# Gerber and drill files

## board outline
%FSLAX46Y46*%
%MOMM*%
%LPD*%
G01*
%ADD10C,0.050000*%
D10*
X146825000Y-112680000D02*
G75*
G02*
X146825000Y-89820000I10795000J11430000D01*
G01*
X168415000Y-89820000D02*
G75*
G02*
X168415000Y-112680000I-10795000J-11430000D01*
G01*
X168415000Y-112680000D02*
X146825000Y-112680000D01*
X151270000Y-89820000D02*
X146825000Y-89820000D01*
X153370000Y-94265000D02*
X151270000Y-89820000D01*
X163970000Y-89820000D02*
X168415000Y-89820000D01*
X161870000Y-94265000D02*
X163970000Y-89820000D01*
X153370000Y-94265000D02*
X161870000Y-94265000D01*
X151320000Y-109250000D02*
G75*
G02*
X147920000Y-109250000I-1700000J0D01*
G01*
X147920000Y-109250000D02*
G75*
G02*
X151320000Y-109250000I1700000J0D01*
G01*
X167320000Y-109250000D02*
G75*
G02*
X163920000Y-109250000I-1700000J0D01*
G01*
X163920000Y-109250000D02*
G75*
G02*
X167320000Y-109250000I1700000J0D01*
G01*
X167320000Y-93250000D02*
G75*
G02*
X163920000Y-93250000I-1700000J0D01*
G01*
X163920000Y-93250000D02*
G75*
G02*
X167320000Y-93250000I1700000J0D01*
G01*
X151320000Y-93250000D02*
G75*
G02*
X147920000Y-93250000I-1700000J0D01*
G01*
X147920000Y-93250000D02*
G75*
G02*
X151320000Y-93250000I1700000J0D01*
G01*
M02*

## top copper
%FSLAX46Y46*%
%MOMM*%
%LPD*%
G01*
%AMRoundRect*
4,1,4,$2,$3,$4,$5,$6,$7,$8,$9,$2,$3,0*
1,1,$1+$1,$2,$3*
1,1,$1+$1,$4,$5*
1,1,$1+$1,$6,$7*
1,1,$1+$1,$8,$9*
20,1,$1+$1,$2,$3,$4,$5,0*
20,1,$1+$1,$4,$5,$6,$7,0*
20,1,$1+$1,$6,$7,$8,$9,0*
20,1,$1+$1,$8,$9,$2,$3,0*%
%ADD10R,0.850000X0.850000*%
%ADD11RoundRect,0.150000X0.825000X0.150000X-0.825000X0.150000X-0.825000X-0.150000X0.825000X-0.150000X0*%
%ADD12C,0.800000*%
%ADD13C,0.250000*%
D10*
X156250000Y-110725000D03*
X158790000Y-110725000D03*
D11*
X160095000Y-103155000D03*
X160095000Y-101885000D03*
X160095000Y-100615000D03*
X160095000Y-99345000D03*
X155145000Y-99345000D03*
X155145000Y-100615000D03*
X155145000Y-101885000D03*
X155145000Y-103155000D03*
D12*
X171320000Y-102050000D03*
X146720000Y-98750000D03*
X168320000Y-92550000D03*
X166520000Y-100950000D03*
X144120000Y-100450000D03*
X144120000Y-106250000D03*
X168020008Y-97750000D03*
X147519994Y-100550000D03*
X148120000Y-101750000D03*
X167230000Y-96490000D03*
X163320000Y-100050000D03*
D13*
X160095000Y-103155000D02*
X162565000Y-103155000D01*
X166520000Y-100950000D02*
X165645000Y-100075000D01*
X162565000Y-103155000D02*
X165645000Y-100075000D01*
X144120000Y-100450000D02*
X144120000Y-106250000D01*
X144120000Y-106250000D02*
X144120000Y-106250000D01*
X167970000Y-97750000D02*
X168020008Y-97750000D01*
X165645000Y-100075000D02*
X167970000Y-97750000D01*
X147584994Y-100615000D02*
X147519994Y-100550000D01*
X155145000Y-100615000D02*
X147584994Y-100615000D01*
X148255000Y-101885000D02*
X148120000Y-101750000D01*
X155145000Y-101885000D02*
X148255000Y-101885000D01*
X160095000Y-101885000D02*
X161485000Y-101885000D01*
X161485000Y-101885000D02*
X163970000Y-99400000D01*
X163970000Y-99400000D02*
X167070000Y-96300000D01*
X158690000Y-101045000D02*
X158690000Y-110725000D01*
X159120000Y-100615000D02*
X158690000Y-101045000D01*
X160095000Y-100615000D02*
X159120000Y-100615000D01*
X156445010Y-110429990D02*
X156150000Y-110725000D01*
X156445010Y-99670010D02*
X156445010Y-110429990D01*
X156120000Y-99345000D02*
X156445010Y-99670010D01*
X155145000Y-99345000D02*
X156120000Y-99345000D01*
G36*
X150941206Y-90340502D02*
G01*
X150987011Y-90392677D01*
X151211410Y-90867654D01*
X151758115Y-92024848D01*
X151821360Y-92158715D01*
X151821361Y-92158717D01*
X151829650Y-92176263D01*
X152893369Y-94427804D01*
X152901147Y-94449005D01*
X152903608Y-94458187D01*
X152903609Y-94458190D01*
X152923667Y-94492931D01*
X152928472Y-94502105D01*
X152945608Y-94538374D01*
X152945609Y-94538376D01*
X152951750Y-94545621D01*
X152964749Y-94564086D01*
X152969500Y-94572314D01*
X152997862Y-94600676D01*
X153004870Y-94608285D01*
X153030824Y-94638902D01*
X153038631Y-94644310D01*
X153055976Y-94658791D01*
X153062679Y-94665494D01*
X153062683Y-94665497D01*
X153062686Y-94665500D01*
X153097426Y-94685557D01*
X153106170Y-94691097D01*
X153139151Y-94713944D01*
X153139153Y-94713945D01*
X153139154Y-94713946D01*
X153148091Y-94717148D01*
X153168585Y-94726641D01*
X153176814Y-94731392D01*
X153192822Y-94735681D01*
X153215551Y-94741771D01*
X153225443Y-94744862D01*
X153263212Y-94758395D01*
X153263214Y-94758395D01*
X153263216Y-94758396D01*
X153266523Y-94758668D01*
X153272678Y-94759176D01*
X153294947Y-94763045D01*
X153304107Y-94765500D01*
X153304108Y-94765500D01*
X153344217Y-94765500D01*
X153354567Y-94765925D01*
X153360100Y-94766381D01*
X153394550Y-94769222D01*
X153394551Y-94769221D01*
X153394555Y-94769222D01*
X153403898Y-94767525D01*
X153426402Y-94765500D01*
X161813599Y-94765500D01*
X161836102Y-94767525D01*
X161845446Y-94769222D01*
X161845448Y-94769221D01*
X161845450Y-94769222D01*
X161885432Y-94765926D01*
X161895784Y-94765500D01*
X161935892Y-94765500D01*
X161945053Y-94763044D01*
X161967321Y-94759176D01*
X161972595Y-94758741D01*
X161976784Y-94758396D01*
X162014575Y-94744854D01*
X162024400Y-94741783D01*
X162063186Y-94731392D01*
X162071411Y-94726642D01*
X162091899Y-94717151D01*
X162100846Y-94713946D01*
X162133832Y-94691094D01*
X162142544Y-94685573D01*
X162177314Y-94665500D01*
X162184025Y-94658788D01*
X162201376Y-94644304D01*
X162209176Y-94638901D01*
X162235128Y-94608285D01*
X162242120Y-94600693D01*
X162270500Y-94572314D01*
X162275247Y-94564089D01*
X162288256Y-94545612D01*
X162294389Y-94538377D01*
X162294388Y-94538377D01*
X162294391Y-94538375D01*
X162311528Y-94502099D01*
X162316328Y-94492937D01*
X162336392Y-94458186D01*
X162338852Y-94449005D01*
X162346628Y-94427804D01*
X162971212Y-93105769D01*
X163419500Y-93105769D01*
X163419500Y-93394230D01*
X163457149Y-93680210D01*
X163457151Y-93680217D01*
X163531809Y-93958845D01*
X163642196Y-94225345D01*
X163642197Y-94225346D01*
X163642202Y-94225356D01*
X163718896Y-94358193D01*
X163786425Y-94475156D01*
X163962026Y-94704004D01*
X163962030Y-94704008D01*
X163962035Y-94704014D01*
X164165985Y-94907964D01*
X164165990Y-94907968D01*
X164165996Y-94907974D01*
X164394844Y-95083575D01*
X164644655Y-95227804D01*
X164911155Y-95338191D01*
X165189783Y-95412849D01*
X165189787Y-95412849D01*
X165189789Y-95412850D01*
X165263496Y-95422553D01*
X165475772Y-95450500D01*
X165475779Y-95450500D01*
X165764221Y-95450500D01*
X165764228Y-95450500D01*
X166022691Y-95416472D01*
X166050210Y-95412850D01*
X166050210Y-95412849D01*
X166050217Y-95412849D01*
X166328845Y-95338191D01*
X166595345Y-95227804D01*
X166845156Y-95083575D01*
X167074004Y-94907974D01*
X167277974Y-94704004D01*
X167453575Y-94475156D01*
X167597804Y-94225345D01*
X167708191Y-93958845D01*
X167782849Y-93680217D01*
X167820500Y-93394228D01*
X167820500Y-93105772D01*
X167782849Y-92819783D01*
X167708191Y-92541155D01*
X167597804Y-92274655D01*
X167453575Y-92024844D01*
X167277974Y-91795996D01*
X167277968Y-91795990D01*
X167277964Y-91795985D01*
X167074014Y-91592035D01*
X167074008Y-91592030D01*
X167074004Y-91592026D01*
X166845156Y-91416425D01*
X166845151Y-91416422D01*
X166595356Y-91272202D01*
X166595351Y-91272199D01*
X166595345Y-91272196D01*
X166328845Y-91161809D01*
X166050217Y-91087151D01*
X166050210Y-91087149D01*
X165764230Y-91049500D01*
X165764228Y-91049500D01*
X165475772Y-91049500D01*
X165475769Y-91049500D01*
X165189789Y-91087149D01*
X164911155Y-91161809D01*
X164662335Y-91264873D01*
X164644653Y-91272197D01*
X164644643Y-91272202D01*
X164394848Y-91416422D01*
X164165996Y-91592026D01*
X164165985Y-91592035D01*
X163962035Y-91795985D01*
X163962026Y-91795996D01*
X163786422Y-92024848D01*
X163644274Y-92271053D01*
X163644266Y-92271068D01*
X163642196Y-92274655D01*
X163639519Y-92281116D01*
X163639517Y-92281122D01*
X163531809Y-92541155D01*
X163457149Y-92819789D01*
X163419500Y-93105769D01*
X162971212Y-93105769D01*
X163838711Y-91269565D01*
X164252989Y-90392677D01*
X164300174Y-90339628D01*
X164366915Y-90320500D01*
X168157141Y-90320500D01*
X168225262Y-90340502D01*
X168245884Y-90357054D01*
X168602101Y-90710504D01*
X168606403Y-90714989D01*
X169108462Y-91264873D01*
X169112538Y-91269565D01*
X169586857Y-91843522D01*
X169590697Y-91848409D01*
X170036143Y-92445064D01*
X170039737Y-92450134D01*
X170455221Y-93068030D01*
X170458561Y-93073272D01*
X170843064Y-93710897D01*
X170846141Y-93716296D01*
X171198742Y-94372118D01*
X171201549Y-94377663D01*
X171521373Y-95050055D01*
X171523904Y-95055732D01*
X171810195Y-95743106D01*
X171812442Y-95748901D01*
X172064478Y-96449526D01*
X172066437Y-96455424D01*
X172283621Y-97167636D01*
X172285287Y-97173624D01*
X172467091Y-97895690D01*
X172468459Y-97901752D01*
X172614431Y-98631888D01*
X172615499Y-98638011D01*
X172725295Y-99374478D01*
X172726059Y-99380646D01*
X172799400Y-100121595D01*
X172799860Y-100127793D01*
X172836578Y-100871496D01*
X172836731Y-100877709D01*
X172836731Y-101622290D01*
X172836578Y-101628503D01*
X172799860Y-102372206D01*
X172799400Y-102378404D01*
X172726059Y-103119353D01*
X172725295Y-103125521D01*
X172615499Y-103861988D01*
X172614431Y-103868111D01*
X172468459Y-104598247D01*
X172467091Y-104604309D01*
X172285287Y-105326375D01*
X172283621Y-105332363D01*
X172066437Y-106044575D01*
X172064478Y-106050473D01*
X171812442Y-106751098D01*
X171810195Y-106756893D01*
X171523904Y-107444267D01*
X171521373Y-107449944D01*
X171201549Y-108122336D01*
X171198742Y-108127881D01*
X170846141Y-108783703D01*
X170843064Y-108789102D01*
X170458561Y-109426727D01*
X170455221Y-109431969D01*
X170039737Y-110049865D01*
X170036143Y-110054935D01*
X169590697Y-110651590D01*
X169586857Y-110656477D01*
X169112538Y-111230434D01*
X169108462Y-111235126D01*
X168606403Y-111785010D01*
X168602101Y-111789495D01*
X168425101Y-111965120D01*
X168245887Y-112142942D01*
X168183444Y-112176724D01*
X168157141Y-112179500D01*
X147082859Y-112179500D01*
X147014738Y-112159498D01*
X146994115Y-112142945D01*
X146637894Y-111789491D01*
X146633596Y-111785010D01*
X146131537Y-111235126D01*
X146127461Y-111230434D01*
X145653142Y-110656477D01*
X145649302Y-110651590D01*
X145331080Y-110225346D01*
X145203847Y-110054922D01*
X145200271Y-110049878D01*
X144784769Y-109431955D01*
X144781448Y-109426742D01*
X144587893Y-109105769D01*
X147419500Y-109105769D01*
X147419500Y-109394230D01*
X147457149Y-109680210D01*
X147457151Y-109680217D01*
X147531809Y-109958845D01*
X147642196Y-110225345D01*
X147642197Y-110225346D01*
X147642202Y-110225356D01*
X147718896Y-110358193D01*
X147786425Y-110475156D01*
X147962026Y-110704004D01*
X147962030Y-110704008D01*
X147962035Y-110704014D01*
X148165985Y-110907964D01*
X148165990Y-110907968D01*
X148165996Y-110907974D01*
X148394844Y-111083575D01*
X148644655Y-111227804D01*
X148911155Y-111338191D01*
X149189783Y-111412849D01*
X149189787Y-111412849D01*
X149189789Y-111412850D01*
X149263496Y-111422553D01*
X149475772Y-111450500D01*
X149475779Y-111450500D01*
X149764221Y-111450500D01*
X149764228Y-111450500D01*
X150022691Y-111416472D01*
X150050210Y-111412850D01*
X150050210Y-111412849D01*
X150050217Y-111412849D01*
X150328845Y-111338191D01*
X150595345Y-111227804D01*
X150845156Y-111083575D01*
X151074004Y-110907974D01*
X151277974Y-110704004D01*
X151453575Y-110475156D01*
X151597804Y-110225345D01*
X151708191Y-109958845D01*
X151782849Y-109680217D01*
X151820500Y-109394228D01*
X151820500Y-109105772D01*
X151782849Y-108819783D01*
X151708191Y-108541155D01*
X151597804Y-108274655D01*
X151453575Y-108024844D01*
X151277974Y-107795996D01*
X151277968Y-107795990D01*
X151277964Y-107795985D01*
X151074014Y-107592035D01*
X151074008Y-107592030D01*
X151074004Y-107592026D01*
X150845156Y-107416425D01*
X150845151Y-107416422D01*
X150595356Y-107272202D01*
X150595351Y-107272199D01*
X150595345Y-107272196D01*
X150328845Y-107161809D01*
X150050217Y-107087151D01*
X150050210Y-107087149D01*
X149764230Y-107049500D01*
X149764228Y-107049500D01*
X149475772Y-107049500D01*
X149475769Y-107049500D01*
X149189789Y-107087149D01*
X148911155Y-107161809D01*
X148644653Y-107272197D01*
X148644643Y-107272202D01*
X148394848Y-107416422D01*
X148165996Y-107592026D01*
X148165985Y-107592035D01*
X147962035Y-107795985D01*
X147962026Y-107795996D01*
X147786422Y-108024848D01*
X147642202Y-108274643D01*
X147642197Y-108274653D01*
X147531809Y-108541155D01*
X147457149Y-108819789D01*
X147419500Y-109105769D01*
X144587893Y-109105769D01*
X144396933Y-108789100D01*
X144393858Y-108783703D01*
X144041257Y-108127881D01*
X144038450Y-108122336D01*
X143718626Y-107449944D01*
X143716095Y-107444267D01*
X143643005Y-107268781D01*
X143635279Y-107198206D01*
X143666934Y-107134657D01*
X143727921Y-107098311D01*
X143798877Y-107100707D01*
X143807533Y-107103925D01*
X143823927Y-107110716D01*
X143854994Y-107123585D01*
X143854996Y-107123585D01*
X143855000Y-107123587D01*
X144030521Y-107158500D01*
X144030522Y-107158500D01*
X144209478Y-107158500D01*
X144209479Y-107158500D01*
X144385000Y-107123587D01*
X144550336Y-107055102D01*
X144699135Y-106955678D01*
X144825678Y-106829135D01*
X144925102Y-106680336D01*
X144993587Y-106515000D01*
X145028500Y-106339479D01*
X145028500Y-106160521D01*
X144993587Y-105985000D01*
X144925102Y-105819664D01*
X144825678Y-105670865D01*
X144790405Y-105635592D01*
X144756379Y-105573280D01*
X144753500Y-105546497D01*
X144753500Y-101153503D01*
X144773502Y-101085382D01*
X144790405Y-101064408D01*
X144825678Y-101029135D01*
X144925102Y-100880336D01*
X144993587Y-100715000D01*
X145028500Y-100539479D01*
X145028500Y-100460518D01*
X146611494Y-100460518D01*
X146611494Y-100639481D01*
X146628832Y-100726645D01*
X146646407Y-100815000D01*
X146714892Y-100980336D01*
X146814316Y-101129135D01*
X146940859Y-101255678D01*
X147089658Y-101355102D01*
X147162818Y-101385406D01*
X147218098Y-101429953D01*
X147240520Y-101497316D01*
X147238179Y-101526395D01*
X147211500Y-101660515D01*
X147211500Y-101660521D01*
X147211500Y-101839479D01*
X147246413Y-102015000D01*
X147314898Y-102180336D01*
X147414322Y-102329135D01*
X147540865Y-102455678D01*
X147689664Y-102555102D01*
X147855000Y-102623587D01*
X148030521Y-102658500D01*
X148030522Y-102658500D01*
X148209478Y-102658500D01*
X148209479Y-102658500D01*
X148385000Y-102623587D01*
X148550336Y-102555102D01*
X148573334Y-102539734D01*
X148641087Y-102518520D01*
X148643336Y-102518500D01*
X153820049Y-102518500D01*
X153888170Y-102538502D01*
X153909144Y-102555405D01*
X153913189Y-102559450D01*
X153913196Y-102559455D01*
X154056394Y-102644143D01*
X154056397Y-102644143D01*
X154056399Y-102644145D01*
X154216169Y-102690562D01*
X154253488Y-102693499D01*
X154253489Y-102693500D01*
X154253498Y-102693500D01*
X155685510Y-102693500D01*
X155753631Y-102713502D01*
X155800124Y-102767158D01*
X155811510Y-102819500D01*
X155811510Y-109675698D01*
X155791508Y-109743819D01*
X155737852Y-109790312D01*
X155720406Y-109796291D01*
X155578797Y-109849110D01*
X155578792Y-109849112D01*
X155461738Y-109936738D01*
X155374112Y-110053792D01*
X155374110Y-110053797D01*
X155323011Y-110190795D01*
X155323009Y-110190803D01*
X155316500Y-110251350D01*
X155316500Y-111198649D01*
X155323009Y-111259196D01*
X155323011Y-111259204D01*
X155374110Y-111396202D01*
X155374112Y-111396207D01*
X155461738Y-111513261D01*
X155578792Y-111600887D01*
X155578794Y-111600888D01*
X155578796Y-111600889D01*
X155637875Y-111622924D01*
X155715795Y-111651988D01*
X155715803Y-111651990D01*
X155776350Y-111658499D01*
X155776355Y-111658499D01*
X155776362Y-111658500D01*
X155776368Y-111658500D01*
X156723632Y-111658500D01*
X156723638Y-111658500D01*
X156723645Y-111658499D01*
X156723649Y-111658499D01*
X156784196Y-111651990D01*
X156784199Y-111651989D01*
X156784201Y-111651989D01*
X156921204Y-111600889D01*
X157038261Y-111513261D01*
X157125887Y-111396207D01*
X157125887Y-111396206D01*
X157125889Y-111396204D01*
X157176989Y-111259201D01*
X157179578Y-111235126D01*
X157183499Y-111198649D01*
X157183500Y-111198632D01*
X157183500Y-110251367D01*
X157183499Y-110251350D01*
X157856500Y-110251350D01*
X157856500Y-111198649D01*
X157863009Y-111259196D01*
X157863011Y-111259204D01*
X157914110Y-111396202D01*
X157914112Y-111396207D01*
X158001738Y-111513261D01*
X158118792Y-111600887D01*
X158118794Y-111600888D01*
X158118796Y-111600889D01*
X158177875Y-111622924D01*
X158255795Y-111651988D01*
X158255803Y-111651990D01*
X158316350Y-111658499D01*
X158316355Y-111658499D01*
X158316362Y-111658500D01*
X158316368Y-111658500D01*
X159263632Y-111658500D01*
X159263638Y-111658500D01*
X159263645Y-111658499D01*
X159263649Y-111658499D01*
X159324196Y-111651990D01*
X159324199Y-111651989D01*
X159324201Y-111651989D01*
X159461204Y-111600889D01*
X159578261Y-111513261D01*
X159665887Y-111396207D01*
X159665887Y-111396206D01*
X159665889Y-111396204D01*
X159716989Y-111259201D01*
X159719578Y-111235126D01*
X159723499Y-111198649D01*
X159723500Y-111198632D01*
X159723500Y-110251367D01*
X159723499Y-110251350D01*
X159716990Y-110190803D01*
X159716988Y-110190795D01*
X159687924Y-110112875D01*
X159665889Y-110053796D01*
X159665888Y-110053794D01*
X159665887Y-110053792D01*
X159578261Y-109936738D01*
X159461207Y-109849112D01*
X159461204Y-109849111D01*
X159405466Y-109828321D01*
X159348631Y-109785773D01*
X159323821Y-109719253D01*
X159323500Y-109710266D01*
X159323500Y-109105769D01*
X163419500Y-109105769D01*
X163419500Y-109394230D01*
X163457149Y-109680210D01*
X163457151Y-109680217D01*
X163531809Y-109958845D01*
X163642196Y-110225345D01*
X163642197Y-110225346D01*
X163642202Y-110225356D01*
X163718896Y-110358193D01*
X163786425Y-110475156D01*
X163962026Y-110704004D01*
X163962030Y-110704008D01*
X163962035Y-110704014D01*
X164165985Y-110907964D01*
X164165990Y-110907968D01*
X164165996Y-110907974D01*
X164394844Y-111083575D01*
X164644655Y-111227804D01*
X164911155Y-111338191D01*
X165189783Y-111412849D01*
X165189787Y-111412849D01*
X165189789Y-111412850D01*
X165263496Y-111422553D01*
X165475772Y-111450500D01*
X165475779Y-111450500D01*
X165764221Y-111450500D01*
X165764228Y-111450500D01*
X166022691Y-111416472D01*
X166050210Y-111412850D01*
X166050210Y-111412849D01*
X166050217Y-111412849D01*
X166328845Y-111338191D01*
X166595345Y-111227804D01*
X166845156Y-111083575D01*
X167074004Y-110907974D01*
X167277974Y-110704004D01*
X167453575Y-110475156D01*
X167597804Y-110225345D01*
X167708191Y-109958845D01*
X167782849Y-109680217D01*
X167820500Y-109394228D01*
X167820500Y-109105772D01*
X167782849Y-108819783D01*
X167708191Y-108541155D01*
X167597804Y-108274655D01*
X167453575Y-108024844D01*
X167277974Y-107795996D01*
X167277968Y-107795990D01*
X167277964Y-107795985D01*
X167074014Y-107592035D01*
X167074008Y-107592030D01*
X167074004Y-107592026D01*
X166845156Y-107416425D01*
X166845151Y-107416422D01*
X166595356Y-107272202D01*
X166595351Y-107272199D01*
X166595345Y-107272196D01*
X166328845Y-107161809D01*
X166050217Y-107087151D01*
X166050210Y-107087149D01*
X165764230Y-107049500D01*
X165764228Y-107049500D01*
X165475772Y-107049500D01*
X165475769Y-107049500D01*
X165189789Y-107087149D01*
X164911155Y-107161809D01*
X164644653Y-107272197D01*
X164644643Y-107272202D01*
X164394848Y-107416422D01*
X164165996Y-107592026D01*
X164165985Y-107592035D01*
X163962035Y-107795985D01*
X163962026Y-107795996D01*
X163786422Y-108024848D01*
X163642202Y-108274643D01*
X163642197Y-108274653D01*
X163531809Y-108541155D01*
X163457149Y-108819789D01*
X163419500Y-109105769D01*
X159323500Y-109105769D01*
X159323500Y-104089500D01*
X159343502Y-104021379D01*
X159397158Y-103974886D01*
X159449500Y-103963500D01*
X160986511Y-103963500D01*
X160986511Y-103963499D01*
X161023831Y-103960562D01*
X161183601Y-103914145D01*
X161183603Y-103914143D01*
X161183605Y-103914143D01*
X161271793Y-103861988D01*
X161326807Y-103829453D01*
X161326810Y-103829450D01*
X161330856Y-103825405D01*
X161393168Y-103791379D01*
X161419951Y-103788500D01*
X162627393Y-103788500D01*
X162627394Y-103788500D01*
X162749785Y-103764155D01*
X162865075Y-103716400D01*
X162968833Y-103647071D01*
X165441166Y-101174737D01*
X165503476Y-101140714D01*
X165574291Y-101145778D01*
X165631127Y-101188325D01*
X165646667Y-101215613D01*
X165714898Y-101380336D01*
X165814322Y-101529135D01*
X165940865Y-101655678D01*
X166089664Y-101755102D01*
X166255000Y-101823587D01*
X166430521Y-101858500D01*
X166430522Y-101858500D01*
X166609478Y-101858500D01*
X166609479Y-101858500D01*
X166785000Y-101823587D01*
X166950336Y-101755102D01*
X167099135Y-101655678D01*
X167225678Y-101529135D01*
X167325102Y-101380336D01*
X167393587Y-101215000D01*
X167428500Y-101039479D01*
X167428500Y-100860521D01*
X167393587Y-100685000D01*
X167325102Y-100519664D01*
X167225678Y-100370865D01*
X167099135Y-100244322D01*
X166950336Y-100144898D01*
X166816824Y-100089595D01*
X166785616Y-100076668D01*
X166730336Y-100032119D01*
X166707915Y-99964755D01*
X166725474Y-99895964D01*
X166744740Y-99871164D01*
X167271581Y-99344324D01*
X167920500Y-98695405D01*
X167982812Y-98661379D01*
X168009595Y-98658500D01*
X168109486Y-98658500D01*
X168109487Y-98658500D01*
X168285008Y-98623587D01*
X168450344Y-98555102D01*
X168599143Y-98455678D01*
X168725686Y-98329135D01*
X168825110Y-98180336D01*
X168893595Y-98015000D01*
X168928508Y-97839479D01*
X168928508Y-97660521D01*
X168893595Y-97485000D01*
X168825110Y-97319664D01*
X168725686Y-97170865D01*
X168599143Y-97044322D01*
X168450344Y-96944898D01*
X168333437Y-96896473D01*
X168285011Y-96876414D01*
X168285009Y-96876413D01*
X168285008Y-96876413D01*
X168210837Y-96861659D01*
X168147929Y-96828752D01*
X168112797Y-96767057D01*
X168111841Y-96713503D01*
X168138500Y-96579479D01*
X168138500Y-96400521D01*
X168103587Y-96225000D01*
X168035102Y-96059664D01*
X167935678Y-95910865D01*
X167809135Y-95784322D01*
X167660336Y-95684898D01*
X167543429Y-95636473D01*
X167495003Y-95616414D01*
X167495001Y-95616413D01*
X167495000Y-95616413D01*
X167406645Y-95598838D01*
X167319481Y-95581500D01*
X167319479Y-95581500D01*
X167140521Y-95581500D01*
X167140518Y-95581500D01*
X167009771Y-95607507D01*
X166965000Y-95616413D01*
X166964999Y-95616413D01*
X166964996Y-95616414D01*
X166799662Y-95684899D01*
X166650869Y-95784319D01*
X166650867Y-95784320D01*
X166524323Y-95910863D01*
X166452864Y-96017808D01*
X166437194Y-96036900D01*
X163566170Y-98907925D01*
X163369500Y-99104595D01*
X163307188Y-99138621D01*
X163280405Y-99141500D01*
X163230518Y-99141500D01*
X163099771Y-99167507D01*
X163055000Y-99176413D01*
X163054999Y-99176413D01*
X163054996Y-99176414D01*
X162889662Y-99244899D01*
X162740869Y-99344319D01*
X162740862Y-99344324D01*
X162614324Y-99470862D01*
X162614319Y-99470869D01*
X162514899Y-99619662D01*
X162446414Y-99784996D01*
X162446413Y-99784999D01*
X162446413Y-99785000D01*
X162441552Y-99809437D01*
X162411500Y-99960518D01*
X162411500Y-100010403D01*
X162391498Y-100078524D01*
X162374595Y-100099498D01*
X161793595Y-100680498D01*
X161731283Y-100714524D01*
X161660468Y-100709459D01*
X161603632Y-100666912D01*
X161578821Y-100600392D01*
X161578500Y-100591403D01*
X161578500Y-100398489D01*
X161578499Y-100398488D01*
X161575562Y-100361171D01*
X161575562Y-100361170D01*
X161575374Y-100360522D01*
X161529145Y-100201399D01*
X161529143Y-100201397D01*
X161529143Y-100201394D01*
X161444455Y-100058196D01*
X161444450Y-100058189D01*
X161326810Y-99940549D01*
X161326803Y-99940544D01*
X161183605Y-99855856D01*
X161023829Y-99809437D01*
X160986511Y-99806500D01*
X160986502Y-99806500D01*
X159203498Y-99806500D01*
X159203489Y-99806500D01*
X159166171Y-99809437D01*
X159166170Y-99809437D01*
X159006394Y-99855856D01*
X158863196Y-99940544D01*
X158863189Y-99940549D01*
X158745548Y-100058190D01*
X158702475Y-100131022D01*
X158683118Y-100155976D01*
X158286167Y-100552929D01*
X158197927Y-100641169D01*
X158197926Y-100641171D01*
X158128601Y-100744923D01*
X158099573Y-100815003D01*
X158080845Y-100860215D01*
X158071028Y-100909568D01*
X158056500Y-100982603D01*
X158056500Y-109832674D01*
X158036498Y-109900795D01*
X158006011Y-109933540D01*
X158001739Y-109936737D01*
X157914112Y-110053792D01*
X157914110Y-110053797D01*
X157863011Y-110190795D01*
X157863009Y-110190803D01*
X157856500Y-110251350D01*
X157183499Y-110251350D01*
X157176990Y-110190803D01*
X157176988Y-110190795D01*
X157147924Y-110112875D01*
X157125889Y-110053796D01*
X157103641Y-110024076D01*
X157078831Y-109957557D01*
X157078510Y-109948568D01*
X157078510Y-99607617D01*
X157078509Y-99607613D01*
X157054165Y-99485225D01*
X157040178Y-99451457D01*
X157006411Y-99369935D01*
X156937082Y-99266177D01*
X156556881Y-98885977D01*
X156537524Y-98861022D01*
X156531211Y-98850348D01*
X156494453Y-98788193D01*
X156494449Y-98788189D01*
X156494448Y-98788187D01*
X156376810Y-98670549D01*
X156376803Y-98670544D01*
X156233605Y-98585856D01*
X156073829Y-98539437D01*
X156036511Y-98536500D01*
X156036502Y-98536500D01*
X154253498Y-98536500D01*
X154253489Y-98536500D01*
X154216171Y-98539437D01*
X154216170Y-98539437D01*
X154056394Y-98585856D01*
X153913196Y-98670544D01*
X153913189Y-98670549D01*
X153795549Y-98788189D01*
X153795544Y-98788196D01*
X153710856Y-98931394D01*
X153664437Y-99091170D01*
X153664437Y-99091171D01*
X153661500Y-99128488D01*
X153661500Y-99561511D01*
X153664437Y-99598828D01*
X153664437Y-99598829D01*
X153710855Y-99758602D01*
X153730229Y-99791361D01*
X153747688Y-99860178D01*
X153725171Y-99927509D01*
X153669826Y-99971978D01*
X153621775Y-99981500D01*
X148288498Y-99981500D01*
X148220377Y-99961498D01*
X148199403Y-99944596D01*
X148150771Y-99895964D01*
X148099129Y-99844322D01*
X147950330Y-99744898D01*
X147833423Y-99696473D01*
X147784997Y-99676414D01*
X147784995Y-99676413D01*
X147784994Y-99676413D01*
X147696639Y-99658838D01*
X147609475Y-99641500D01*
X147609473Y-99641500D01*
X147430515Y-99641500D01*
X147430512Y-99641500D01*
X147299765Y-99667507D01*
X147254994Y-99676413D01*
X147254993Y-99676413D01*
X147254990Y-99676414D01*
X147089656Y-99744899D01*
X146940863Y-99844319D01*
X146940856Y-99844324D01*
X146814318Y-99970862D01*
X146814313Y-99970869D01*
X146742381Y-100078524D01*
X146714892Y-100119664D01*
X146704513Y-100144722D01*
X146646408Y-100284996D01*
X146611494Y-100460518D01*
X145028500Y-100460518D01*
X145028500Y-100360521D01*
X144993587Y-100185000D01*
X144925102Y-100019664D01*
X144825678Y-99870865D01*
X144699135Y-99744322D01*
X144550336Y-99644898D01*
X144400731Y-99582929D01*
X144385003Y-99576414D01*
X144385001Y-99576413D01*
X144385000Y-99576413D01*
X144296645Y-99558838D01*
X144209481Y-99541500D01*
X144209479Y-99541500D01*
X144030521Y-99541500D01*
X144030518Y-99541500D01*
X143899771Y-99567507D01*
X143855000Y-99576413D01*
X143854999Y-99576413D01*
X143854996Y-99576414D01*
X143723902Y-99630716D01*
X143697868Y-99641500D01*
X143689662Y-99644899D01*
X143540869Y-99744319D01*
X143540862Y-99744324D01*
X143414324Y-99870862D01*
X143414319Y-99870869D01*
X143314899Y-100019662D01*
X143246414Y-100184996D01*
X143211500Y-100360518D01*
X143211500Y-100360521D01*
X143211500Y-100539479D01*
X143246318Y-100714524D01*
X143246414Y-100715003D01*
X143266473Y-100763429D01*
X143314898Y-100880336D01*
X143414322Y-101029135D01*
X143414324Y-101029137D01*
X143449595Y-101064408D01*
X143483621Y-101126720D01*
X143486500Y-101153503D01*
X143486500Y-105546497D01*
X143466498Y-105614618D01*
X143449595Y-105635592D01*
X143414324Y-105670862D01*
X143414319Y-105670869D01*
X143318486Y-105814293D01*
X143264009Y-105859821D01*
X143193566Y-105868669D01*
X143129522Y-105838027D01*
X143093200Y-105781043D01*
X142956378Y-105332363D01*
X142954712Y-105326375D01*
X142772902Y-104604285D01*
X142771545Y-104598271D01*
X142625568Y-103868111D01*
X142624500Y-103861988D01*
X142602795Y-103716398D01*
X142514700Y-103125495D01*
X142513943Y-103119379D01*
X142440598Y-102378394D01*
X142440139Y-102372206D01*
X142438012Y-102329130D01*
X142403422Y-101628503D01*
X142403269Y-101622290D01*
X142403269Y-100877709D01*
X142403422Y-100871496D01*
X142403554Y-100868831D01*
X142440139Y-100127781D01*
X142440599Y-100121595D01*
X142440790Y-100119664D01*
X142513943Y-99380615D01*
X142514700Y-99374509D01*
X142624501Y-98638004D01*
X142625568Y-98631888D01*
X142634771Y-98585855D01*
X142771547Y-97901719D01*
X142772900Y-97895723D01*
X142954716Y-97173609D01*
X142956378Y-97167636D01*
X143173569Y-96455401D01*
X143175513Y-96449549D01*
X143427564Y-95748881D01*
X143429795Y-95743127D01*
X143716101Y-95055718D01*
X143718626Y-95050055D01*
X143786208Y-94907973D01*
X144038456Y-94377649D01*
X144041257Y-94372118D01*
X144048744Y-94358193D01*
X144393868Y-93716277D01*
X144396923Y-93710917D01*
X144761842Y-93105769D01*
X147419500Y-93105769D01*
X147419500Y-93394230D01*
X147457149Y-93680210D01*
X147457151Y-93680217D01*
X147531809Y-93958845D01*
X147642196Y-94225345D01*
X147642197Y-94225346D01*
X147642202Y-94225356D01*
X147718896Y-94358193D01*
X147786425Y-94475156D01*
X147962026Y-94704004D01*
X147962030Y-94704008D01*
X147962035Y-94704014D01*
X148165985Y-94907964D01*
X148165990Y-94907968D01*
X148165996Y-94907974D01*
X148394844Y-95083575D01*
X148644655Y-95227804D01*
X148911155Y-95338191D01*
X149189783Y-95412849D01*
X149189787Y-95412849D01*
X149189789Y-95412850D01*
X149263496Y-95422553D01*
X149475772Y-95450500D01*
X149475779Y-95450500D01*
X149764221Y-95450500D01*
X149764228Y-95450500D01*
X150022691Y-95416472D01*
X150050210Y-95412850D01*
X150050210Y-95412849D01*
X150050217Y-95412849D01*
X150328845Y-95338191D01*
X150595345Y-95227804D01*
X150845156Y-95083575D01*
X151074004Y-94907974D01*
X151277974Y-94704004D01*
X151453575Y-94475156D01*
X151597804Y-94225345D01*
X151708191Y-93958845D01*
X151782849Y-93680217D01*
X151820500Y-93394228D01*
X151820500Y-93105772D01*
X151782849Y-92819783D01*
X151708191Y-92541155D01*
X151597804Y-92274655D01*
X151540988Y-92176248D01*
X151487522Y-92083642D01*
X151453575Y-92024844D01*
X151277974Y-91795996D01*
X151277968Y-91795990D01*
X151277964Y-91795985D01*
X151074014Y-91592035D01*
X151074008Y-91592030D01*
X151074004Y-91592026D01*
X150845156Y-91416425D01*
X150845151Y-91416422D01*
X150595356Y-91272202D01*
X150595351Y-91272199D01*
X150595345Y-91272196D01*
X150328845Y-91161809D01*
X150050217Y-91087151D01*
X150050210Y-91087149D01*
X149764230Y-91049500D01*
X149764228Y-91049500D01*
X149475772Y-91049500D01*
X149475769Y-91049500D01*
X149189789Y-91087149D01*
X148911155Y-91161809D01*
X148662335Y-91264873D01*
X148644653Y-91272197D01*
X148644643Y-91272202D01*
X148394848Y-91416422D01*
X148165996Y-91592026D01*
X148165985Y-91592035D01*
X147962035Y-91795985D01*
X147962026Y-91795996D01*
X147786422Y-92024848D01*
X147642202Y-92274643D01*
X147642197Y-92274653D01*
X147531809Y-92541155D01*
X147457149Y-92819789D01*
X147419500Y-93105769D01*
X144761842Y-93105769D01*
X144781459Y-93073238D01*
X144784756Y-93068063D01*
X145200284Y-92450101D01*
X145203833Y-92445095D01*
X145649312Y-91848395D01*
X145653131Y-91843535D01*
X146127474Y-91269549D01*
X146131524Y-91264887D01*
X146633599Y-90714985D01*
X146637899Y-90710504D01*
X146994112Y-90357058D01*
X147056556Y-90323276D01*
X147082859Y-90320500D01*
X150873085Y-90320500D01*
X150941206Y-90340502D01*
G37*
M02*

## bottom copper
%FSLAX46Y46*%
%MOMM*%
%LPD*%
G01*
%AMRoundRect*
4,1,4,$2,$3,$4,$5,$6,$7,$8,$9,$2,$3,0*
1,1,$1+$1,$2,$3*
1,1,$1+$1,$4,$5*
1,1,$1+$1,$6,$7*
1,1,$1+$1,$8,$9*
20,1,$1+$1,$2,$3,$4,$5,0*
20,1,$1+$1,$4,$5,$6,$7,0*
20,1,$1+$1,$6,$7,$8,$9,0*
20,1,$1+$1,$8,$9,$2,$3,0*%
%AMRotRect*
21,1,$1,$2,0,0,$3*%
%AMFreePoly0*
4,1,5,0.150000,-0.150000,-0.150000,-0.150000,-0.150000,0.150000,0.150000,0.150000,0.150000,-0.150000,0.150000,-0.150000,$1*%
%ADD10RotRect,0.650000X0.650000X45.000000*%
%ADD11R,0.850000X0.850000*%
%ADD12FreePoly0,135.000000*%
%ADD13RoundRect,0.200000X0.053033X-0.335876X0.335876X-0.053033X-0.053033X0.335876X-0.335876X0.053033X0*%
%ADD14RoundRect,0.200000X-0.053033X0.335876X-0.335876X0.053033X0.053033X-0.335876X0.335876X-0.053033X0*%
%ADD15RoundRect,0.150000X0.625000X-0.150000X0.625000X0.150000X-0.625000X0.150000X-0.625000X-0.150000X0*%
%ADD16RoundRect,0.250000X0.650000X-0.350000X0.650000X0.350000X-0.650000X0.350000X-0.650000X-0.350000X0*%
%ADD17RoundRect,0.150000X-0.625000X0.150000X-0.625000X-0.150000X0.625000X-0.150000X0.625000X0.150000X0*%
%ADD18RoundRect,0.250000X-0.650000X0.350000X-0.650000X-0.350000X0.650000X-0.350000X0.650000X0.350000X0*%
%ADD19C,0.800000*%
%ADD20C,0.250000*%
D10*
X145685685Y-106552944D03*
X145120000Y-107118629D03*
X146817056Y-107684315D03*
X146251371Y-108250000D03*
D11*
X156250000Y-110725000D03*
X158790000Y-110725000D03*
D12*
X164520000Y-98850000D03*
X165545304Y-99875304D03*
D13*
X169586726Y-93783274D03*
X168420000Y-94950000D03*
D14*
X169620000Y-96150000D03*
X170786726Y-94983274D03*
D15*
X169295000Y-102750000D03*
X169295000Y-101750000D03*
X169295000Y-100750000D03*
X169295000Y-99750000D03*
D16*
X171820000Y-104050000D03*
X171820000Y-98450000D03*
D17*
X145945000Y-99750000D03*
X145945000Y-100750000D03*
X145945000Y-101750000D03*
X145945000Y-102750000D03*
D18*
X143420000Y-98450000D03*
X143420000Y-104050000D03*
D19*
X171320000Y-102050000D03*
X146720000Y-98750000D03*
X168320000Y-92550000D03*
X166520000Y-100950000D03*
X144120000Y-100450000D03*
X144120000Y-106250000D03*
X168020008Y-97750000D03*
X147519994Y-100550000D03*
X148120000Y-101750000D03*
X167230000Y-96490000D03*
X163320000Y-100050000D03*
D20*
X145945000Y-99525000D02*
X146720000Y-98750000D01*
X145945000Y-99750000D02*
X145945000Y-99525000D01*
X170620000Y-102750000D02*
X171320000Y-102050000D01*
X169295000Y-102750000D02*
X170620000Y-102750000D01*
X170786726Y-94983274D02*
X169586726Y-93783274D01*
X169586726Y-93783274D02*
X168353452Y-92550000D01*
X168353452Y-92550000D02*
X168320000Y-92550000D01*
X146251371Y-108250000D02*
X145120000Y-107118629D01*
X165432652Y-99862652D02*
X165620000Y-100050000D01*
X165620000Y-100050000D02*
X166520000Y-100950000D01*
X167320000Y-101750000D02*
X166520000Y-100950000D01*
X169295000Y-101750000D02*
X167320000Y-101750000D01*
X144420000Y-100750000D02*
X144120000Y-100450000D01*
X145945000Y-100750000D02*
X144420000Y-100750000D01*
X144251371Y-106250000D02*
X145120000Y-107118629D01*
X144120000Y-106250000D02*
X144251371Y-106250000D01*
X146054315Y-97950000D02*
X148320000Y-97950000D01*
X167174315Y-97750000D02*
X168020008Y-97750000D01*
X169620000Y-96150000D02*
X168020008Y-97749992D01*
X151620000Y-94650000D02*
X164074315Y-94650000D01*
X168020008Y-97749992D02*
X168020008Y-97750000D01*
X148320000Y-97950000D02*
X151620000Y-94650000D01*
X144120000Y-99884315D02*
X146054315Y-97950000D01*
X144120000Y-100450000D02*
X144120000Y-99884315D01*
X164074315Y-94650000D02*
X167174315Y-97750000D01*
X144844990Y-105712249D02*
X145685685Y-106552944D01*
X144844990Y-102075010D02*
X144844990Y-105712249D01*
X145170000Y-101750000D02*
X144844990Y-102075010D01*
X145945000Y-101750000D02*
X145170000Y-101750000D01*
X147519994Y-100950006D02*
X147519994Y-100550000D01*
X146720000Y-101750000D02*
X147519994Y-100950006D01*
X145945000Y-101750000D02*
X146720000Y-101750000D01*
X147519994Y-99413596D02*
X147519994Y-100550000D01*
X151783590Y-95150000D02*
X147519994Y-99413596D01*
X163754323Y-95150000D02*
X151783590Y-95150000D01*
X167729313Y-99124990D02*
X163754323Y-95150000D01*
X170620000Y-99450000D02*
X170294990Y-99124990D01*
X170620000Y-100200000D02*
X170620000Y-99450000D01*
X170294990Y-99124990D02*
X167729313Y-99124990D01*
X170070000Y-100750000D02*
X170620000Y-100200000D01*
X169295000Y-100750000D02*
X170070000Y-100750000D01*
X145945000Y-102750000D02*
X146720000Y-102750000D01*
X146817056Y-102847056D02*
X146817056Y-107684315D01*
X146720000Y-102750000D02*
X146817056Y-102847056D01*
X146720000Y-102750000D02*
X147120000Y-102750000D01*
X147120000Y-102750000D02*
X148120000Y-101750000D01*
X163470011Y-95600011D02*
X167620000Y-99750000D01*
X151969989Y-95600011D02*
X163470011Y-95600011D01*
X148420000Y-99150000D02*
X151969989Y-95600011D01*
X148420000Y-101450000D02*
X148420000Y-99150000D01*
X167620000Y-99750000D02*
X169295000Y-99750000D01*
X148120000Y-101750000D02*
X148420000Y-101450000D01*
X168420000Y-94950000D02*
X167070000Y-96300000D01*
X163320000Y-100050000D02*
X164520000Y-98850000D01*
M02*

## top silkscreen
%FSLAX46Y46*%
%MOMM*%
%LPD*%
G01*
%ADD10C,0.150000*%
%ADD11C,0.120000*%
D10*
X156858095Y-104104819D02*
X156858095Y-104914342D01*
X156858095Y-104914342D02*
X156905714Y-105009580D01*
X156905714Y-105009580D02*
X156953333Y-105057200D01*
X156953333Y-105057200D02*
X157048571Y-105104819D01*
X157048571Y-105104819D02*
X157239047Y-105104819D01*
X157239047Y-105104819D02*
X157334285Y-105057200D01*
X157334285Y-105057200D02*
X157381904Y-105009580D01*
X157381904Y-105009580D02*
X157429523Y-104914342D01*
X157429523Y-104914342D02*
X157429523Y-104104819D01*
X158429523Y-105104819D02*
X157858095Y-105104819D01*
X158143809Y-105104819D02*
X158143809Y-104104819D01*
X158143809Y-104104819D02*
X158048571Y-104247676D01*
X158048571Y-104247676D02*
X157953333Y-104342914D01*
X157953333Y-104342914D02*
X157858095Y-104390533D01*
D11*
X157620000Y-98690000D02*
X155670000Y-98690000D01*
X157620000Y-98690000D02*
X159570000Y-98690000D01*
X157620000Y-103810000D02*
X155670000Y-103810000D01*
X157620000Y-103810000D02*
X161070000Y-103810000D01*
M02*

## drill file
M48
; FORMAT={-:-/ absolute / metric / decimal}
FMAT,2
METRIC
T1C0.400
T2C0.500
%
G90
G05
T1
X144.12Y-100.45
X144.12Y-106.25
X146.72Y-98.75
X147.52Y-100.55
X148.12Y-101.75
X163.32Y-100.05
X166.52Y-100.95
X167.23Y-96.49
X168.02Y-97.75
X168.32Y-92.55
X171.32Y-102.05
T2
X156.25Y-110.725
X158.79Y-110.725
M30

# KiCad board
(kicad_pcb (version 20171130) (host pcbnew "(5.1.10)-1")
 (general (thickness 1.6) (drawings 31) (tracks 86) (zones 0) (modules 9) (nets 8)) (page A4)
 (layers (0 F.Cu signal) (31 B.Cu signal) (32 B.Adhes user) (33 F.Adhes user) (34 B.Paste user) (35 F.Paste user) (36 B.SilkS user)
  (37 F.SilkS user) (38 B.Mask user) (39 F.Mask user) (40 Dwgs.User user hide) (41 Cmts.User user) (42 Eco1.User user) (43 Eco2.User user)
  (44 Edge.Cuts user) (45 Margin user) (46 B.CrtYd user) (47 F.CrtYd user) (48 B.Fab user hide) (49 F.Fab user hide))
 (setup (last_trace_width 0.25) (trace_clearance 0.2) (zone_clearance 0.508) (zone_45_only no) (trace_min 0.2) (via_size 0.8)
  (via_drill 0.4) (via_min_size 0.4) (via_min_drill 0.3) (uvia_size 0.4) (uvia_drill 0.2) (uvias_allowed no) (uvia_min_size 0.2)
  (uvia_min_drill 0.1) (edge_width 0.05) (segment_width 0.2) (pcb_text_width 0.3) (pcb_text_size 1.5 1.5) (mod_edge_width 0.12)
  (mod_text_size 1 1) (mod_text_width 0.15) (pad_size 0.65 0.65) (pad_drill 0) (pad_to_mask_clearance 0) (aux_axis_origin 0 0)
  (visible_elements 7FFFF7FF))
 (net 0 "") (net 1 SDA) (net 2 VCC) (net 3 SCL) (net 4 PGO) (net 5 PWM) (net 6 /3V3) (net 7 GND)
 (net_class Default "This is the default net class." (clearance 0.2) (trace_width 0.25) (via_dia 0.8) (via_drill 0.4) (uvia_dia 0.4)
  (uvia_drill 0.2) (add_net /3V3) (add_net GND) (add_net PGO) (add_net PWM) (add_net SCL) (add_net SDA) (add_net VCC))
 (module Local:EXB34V (layer B.Cu) (at 145.968528 107.401472 45)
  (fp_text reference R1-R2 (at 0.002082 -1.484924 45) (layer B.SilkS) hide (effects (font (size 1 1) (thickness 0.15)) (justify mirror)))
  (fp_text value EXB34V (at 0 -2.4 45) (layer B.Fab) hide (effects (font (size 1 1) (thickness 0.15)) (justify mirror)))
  (pad 4 smd rect (at 0.4 -0.8 45) (size 0.65 0.65) (layers B.Cu B.Paste B.Mask) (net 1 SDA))
  (pad 3 smd rect (at -0.4 -0.8 45) (size 0.65 0.65) (layers B.Cu B.Paste B.Mask) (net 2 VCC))
  (pad 2 smd rect (at 0.4 0.8 45) (size 0.65 0.65) (layers B.Cu B.Paste B.Mask) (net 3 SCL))
  (pad 1 smd rect (at -0.4 0.8 45) (size 0.65 0.65) (layers B.Cu B.Paste B.Mask) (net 2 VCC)))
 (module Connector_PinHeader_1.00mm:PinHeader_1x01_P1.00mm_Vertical (layer B.Cu) (at 156.25 110.725 270)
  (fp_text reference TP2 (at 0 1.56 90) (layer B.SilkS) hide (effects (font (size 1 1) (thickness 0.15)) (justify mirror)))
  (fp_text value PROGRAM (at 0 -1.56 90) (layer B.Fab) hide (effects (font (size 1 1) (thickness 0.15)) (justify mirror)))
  (pad 1 thru_hole rect (at 0 0 270) (size 0.85 0.85) (drill 0.5) (layers *.Cu *.Mask) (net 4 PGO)))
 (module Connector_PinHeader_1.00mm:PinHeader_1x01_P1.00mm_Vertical (layer B.Cu) (at 158.79 110.725 270)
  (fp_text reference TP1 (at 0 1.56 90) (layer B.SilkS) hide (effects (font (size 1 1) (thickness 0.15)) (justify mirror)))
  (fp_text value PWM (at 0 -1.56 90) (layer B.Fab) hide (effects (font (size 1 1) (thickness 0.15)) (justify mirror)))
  (pad 1 thru_hole rect (at 0 0 270) (size 0.85 0.85) (drill 0.5) (layers *.Cu *.Mask) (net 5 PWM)))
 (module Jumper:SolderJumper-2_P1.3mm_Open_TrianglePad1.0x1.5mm (layer B.Cu) (at 165.032652 99.362652 135)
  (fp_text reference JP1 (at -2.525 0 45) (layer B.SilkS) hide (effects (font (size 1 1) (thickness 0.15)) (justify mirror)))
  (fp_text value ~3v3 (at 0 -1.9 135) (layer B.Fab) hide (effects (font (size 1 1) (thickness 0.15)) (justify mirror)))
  (pad 2 smd custom (at 0.725 0 135) (size 0.3 0.3) (layers B.Cu B.Mask) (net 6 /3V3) (zone_connect 2)
   (options (clearance outline) (anchor rect)) (primitives))
  (pad 1 smd custom (at -0.725 0 135) (size 0.3 0.3) (layers B.Cu B.Mask) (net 2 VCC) (zone_connect 2)
   (options (clearance outline) (anchor rect)) (primitives)))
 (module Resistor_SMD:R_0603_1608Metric (layer B.Cu) (at 169.003363 94.366637 45)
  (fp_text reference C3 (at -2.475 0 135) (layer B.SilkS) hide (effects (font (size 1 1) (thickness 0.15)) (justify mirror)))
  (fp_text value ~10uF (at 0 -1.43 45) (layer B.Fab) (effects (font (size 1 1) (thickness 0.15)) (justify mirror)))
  (pad 2 smd roundrect (at 0.825 0 45) (size 0.8 0.95) (layers B.Cu B.Paste B.Mask) (roundrect_rratio 0.25) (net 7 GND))
  (pad 1 smd roundrect (at -0.825 0 45) (size 0.8 0.95) (layers B.Cu B.Paste B.Mask) (roundrect_rratio 0.25) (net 6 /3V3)))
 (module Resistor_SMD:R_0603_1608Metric (layer B.Cu) (at 170.203363 95.566637 225)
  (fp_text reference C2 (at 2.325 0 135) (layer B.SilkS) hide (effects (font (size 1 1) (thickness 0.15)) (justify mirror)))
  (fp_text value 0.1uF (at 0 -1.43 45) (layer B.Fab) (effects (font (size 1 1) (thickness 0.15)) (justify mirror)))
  (pad 2 smd roundrect (at 0.825 0 225) (size 0.8 0.95) (layers B.Cu B.Paste B.Mask) (roundrect_rratio 0.25) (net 2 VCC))
  (pad 1 smd roundrect (at -0.825 0 225) (size 0.8 0.95) (layers B.Cu B.Paste B.Mask) (roundrect_rratio 0.25) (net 7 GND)))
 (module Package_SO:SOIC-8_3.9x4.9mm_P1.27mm (layer F.Cu) (at 157.62 101.25 180)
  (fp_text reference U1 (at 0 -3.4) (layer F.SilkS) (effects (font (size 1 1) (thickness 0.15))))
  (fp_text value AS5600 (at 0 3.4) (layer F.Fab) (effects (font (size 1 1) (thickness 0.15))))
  (fp_line (start 0 2.56) (end 1.95 2.56) (layer F.SilkS) (width 0.12))
  (fp_line (start 0 2.56) (end -1.95 2.56) (layer F.SilkS) (width 0.12))
  (fp_line (start 0 -2.56) (end 1.95 -2.56) (layer F.SilkS) (width 0.12))
  (fp_line (start 0 -2.56) (end -3.45 -2.56) (layer F.SilkS) (width 0.12))
  (pad 1 smd roundrect (at -2.475 -1.905 180) (size 1.95 0.6) (layers F.Cu F.Paste F.Mask) (roundrect_rratio 0.25) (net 2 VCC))
  (pad 2 smd roundrect (at -2.475 -0.635 180) (size 1.95 0.6) (layers F.Cu F.Paste F.Mask) (roundrect_rratio 0.25) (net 6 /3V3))
  (pad 3 smd roundrect (at -2.475 0.635 180) (size 1.95 0.6) (layers F.Cu F.Paste F.Mask) (roundrect_rratio 0.25) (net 5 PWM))
  (pad 4 smd roundrect (at -2.475 1.905 180) (size 1.95 0.6) (layers F.Cu F.Paste F.Mask) (roundrect_rratio 0.25) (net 7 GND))
  (pad 5 smd roundrect (at 2.475 1.905 180) (size 1.95 0.6) (layers F.Cu F.Paste F.Mask) (roundrect_rratio 0.25) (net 4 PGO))
  (pad 6 smd roundrect (at 2.475 0.635 180) (size 1.95 0.6) (layers F.Cu F.Paste F.Mask) (roundrect_rratio 0.25) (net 1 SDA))
  (pad 7 smd roundrect (at 2.475 -0.635 180) (size 1.95 0.6) (layers F.Cu F.Paste F.Mask) (roundrect_rratio 0.25) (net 3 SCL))
  (pad 8 smd roundrect (at 2.475 -1.905 180) (size 1.95 0.6) (layers F.Cu F.Paste F.Mask) (roundrect_rratio 0.25) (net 7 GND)))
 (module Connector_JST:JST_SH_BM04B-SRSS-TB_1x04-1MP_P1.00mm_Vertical (layer B.Cu) (at 170.62 101.25 90)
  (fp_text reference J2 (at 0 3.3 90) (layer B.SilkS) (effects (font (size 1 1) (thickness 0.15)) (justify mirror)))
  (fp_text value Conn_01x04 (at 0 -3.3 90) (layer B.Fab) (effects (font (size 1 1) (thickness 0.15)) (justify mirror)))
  (pad 1 smd roundrect (at -1.5 -1.325 90) (size 0.6 1.55) (layers B.Cu B.Paste B.Mask) (roundrect_rratio 0.25) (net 7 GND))
  (pad 2 smd roundrect (at -0.5 -1.325 90) (size 0.6 1.55) (layers B.Cu B.Paste B.Mask) (roundrect_rratio 0.25) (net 2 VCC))
  (pad 3 smd roundrect (at 0.5 -1.325 90) (size 0.6 1.55) (layers B.Cu B.Paste B.Mask) (roundrect_rratio 0.25) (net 1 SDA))
  (pad 4 smd roundrect (at 1.5 -1.325 90) (size 0.6 1.55) (layers B.Cu B.Paste B.Mask) (roundrect_rratio 0.25) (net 3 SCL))
  (pad MP smd roundrect (at -2.8 1.2 90) (size 1.2 1.8) (layers B.Cu B.Paste B.Mask) (roundrect_rratio 0.208333))
  (pad MP smd roundrect (at 2.8 1.2 90) (size 1.2 1.8) (layers B.Cu B.Paste B.Mask) (roundrect_rratio 0.208333)))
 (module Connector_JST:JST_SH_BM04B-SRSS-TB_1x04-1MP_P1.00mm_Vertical (layer B.Cu) (at 144.62 101.25 270)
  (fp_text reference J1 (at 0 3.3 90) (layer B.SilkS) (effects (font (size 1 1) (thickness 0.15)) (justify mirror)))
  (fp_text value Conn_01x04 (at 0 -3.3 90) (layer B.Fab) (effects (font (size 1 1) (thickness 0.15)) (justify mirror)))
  (pad 1 smd roundrect (at -1.5 -1.325 270) (size 0.6 1.55) (layers B.Cu B.Paste B.Mask) (roundrect_rratio 0.25) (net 7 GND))
  (pad 2 smd roundrect (at -0.5 -1.325 270) (size 0.6 1.55) (layers B.Cu B.Paste B.Mask) (roundrect_rratio 0.25) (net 2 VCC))
  (pad 3 smd roundrect (at 0.5 -1.325 270) (size 0.6 1.55) (layers B.Cu B.Paste B.Mask) (roundrect_rratio 0.25) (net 1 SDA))
  (pad 4 smd roundrect (at 1.5 -1.325 270) (size 0.6 1.55) (layers B.Cu B.Paste B.Mask) (roundrect_rratio 0.25) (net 3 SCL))
  (pad MP smd roundrect (at -2.8 1.2 270) (size 1.2 1.8) (layers B.Cu B.Paste B.Mask) (roundrect_rratio 0.208333))
  (pad MP smd roundrect (at 2.8 1.2 270) (size 1.2 1.8) (layers B.Cu B.Paste B.Mask) (roundrect_rratio 0.208333)))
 (gr_arc (start 157.62 101.25) (end 146.825 89.82) (angle -93.27315408) (layer Edge.Cuts) (width 0.05))
 (gr_arc (start 157.62 101.25) (end 168.415 112.68) (angle -93.27315408) (layer Edge.Cuts) (width 0.05))
 (gr_line (start 168.415 112.68) (end 146.825 112.68) (layer Edge.Cuts) (width 0.05))
 (gr_line (start 151.27 89.82) (end 146.825 89.82) (layer Edge.Cuts) (width 0.05))
 (gr_line (start 153.37 94.265) (end 151.27 89.82) (layer Edge.Cuts) (width 0.05))
 (gr_line (start 163.97 89.82) (end 168.415 89.82) (layer Edge.Cuts) (width 0.05))
 (gr_line (start 161.87 94.265) (end 163.97 89.82) (layer Edge.Cuts) (width 0.05))
 (gr_line (start 153.37 94.265) (end 161.87 94.265) (layer Edge.Cuts) (width 0.05))
 (gr_circle (center 149.62 109.25) (end 151.32 109.25) (layer Edge.Cuts) (width 0.05))
 (gr_circle (center 165.62 109.25) (end 167.32 109.25) (layer Edge.Cuts) (width 0.05))
 (gr_circle (center 165.62 93.25) (end 167.32 93.25) (layer Edge.Cuts) (width 0.05))
 (gr_circle (center 149.62 93.25) (end 151.32 93.25) (layer Edge.Cuts) (width 0.05))
 (via (at 171.32 102.05) (size 0.8) (drill 0.4) (layers F.Cu B.Cu) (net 7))
 (via (at 146.72 98.75) (size 0.8) (drill 0.4) (layers F.Cu B.Cu) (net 7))
 (segment (start 145.945 99.525) (end 146.72 98.75) (width 0.25) (layer B.Cu) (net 7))
 (segment (start 145.945 99.75) (end 145.945 99.525) (width 0.25) (layer B.Cu) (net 7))
 (segment (start 170.62 102.75) (end 171.32 102.05) (width 0.25) (layer B.Cu) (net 7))
 (segment (start 169.295 102.75) (end 170.62 102.75) (width 0.25) (layer B.Cu) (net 7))
 (segment (start 170.786726 94.983274) (end 169.586726 93.783274) (width 0.25) (layer B.Cu) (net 7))
 (via (at 168.32 92.55) (size 0.8) (drill 0.4) (layers F.Cu B.Cu) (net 7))
 (segment (start 169.586726 93.783274) (end 168.353452 92.55) (width 0.25) (layer B.Cu) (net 7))
 (segment (start 168.353452 92.55) (end 168.32 92.55) (width 0.25) (layer B.Cu) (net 7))
 (segment (start 146.251371 108.25) (end 145.12 107.118629) (width 0.25) (layer B.Cu) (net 2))
 (segment (start 160.095 103.155) (end 162.565 103.155) (width 0.25) (layer F.Cu) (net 2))
 (via (at 166.52 100.95) (size 0.8) (drill 0.4) (layers F.Cu B.Cu) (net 2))
 (segment (start 165.432652 99.862652) (end 165.62 100.05) (width 0.25) (layer B.Cu) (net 2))
 (segment (start 165.62 100.05) (end 166.52 100.95) (width 0.25) (layer B.Cu) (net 2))
 (segment (start 167.32 101.75) (end 166.52 100.95) (width 0.25) (layer B.Cu) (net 2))
 (segment (start 169.295 101.75) (end 167.32 101.75) (width 0.25) (layer B.Cu) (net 2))
 (segment (start 166.52 100.95) (end 165.645 100.075) (width 0.25) (layer F.Cu) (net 2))
 (segment (start 162.565 103.155) (end 165.645 100.075) (width 0.25) (layer F.Cu) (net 2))
 (segment (start 144.42 100.75) (end 144.12 100.45) (width 0.25) (layer B.Cu) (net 2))
 (segment (start 145.945 100.75) (end 144.42 100.75) (width 0.25) (layer B.Cu) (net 2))
 (via (at 144.12 100.45) (size 0.8) (drill 0.4) (layers F.Cu B.Cu) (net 2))
 (segment (start 144.12 100.45) (end 144.12 106.25) (width 0.25) (layer F.Cu) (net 2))
 (segment (start 144.12 106.25) (end 144.12 106.25) (width 0.25) (layer F.Cu) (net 2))
 (via (at 144.12 106.25) (size 0.8) (drill 0.4) (layers F.Cu B.Cu) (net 2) (status 1000000))
 (segment (start 144.251371 106.25) (end 145.12 107.118629) (width 0.25) (layer B.Cu) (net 2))
 (segment (start 144.12 106.25) (end 144.251371 106.25) (width 0.25) (layer B.Cu) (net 2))
 (via (at 168.020008 97.75) (size 0.8) (drill 0.4) (layers F.Cu B.Cu) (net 2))
 (segment (start 146.054315 97.95) (end 148.32 97.95) (width 0.25) (layer B.Cu) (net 2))
 (segment (start 167.174315 97.75) (end 168.020008 97.75) (width 0.25) (layer B.Cu) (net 2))
 (segment (start 169.62 96.15) (end 168.020008 97.749992) (width 0.25) (layer B.Cu) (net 2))
 (segment (start 151.62 94.65) (end 164.074315 94.65) (width 0.25) (layer B.Cu) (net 2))
 (segment (start 168.020008 97.749992) (end 168.020008 97.75) (width 0.25) (layer B.Cu) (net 2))
 (segment (start 148.32 97.95) (end 151.62 94.65) (width 0.25) (layer B.Cu) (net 2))
 (segment (start 144.12 99.884315) (end 146.054315 97.95) (width 0.25) (layer B.Cu) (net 2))
 (segment (start 144.12 100.45) (end 144.12 99.884315) (width 0.25) (layer B.Cu) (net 2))
 (segment (start 167.97 97.75) (end 168.020008 97.75) (width 0.25) (layer F.Cu) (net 2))
 (segment (start 164.074315 94.65) (end 167.174315 97.75) (width 0.25) (layer B.Cu) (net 2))
 (segment (start 165.645 100.075) (end 167.97 97.75) (width 0.25) (layer F.Cu) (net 2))
 (segment (start 144.84499 105.712249) (end 145.685685 106.552944) (width 0.25) (layer B.Cu) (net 1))
 (segment (start 144.84499 102.07501) (end 144.84499 105.712249) (width 0.25) (layer B.Cu) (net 1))
 (segment (start 145.17 101.75) (end 144.84499 102.07501) (width 0.25) (layer B.Cu) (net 1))
 (segment (start 145.945 101.75) (end 145.17 101.75) (width 0.25) (layer B.Cu) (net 1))
 (via (at 147.519994 100.55) (size 0.8) (drill 0.4) (layers F.Cu B.Cu) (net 1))
 (segment (start 147.519994 100.950006) (end 147.519994 100.55) (width 0.25) (layer B.Cu) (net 1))
 (segment (start 146.72 101.75) (end 147.519994 100.950006) (width 0.25) (layer B.Cu) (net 1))
 (segment (start 145.945 101.75) (end 146.72 101.75) (width 0.25) (layer B.Cu) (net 1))
 (segment (start 147.584994 100.615) (end 147.519994 100.55) (width 0.25) (layer F.Cu) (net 1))
 (segment (start 155.145 100.615) (end 147.584994 100.615) (width 0.25) (layer F.Cu) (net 1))
 (segment (start 147.519994 99.413596) (end 147.519994 100.55) (width 0.25) (layer B.Cu) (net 1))
 (segment (start 151.78359 95.15) (end 147.519994 99.413596) (width 0.25) (layer B.Cu) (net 1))
 (segment (start 163.754323 95.15) (end 151.78359 95.15) (width 0.25) (layer B.Cu) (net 1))
 (segment (start 167.729313 99.12499) (end 163.754323 95.15) (width 0.25) (layer B.Cu) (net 1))
 (segment (start 170.62 99.45) (end 170.29499 99.12499) (width 0.25) (layer B.Cu) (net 1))
 (segment (start 170.62 100.2) (end 170.62 99.45) (width 0.25) (layer B.Cu) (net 1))
 (segment (start 170.29499 99.12499) (end 167.729313 99.12499) (width 0.25) (layer B.Cu) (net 1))
 (segment (start 170.07 100.75) (end 170.62 100.2) (width 0.25) (layer B.Cu) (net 1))
 (segment (start 169.295 100.75) (end 170.07 100.75) (width 0.25) (layer B.Cu) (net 1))
 (segment (start 145.945 102.75) (end 146.72 102.75) (width 0.25) (layer B.Cu) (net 3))
 (segment (start 146.817056 102.847056) (end 146.817056 107.684315) (width 0.25) (layer B.Cu) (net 3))
 (segment (start 146.72 102.75) (end 146.817056 102.847056) (width 0.25) (layer B.Cu) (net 3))
 (via (at 148.12 101.75) (size 0.8) (drill 0.4) (layers F.Cu B.Cu) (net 3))
 (segment (start 148.255 101.885) (end 148.12 101.75) (width 0.25) (layer F.Cu) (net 3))
 (segment (start 146.72 102.75) (end 147.12 102.75) (width 0.25) (layer B.Cu) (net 3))
 (segment (start 147.12 102.75) (end 148.12 101.75) (width 0.25) (layer B.Cu) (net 3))
 (segment (start 155.145 101.885) (end 148.255 101.885) (width 0.25) (layer F.Cu) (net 3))
 (segment (start 163.470011 95.600011) (end 167.62 99.75) (width 0.25) (layer B.Cu) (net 3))
 (segment (start 151.969989 95.600011) (end 163.470011 95.600011) (width 0.25) (layer B.Cu) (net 3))
 (segment (start 148.42 99.15) (end 151.969989 95.600011) (width 0.25) (layer B.Cu) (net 3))
 (segment (start 148.42 101.45) (end 148.42 99.15) (width 0.25) (layer B.Cu) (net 3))
 (segment (start 167.62 99.75) (end 169.295 99.75) (width 0.25) (layer B.Cu) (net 3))
 (segment (start 148.12 101.75) (end 148.42 101.45) (width 0.25) (layer B.Cu) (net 3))
 (via (at 167.23 96.49) (size 0.8) (drill 0.4) (layers F.Cu B.Cu) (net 6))
 (segment (start 168.42 94.95) (end 167.07 96.3) (width 0.25) (layer B.Cu) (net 6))
 (segment (start 160.095 101.885) (end 161.485 101.885) (width 0.25) (layer F.Cu) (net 6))
 (segment (start 161.485 101.885) (end 163.97 99.4) (width 0.25) (layer F.Cu) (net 6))
 (segment (start 163.97 99.4) (end 167.07 96.3) (width 0.25) (layer F.Cu) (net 6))
 (via (at 163.32 100.05) (size 0.8) (drill 0.4) (layers F.Cu B.Cu) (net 6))
 (segment (start 163.32 100.05) (end 164.52 98.85) (width 0.25) (layer B.Cu) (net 6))
 (segment (start 158.69 101.045) (end 158.69 110.725) (width 0.25) (layer F.Cu) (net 5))
 (segment (start 159.12 100.615) (end 158.69 101.045) (width 0.25) (layer F.Cu) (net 5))
 (segment (start 160.095 100.615) (end 159.12 100.615) (width 0.25) (layer F.Cu) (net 5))
 (segment (start 156.44501 110.42999) (end 156.15 110.725) (width 0.25) (layer F.Cu) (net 4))
 (segment (start 156.44501 99.67001) (end 156.44501 110.42999) (width 0.25) (layer F.Cu) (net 4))
 (segment (start 156.12 99.345) (end 156.44501 99.67001) (width 0.25) (layer F.Cu) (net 4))
 (segment (start 155.145 99.345) (end 156.12 99.345) (width 0.25) (layer F.Cu) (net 4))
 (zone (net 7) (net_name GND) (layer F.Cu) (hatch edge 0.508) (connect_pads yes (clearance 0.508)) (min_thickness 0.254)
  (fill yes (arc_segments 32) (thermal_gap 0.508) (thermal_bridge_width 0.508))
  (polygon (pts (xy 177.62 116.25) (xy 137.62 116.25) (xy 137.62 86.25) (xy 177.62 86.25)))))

